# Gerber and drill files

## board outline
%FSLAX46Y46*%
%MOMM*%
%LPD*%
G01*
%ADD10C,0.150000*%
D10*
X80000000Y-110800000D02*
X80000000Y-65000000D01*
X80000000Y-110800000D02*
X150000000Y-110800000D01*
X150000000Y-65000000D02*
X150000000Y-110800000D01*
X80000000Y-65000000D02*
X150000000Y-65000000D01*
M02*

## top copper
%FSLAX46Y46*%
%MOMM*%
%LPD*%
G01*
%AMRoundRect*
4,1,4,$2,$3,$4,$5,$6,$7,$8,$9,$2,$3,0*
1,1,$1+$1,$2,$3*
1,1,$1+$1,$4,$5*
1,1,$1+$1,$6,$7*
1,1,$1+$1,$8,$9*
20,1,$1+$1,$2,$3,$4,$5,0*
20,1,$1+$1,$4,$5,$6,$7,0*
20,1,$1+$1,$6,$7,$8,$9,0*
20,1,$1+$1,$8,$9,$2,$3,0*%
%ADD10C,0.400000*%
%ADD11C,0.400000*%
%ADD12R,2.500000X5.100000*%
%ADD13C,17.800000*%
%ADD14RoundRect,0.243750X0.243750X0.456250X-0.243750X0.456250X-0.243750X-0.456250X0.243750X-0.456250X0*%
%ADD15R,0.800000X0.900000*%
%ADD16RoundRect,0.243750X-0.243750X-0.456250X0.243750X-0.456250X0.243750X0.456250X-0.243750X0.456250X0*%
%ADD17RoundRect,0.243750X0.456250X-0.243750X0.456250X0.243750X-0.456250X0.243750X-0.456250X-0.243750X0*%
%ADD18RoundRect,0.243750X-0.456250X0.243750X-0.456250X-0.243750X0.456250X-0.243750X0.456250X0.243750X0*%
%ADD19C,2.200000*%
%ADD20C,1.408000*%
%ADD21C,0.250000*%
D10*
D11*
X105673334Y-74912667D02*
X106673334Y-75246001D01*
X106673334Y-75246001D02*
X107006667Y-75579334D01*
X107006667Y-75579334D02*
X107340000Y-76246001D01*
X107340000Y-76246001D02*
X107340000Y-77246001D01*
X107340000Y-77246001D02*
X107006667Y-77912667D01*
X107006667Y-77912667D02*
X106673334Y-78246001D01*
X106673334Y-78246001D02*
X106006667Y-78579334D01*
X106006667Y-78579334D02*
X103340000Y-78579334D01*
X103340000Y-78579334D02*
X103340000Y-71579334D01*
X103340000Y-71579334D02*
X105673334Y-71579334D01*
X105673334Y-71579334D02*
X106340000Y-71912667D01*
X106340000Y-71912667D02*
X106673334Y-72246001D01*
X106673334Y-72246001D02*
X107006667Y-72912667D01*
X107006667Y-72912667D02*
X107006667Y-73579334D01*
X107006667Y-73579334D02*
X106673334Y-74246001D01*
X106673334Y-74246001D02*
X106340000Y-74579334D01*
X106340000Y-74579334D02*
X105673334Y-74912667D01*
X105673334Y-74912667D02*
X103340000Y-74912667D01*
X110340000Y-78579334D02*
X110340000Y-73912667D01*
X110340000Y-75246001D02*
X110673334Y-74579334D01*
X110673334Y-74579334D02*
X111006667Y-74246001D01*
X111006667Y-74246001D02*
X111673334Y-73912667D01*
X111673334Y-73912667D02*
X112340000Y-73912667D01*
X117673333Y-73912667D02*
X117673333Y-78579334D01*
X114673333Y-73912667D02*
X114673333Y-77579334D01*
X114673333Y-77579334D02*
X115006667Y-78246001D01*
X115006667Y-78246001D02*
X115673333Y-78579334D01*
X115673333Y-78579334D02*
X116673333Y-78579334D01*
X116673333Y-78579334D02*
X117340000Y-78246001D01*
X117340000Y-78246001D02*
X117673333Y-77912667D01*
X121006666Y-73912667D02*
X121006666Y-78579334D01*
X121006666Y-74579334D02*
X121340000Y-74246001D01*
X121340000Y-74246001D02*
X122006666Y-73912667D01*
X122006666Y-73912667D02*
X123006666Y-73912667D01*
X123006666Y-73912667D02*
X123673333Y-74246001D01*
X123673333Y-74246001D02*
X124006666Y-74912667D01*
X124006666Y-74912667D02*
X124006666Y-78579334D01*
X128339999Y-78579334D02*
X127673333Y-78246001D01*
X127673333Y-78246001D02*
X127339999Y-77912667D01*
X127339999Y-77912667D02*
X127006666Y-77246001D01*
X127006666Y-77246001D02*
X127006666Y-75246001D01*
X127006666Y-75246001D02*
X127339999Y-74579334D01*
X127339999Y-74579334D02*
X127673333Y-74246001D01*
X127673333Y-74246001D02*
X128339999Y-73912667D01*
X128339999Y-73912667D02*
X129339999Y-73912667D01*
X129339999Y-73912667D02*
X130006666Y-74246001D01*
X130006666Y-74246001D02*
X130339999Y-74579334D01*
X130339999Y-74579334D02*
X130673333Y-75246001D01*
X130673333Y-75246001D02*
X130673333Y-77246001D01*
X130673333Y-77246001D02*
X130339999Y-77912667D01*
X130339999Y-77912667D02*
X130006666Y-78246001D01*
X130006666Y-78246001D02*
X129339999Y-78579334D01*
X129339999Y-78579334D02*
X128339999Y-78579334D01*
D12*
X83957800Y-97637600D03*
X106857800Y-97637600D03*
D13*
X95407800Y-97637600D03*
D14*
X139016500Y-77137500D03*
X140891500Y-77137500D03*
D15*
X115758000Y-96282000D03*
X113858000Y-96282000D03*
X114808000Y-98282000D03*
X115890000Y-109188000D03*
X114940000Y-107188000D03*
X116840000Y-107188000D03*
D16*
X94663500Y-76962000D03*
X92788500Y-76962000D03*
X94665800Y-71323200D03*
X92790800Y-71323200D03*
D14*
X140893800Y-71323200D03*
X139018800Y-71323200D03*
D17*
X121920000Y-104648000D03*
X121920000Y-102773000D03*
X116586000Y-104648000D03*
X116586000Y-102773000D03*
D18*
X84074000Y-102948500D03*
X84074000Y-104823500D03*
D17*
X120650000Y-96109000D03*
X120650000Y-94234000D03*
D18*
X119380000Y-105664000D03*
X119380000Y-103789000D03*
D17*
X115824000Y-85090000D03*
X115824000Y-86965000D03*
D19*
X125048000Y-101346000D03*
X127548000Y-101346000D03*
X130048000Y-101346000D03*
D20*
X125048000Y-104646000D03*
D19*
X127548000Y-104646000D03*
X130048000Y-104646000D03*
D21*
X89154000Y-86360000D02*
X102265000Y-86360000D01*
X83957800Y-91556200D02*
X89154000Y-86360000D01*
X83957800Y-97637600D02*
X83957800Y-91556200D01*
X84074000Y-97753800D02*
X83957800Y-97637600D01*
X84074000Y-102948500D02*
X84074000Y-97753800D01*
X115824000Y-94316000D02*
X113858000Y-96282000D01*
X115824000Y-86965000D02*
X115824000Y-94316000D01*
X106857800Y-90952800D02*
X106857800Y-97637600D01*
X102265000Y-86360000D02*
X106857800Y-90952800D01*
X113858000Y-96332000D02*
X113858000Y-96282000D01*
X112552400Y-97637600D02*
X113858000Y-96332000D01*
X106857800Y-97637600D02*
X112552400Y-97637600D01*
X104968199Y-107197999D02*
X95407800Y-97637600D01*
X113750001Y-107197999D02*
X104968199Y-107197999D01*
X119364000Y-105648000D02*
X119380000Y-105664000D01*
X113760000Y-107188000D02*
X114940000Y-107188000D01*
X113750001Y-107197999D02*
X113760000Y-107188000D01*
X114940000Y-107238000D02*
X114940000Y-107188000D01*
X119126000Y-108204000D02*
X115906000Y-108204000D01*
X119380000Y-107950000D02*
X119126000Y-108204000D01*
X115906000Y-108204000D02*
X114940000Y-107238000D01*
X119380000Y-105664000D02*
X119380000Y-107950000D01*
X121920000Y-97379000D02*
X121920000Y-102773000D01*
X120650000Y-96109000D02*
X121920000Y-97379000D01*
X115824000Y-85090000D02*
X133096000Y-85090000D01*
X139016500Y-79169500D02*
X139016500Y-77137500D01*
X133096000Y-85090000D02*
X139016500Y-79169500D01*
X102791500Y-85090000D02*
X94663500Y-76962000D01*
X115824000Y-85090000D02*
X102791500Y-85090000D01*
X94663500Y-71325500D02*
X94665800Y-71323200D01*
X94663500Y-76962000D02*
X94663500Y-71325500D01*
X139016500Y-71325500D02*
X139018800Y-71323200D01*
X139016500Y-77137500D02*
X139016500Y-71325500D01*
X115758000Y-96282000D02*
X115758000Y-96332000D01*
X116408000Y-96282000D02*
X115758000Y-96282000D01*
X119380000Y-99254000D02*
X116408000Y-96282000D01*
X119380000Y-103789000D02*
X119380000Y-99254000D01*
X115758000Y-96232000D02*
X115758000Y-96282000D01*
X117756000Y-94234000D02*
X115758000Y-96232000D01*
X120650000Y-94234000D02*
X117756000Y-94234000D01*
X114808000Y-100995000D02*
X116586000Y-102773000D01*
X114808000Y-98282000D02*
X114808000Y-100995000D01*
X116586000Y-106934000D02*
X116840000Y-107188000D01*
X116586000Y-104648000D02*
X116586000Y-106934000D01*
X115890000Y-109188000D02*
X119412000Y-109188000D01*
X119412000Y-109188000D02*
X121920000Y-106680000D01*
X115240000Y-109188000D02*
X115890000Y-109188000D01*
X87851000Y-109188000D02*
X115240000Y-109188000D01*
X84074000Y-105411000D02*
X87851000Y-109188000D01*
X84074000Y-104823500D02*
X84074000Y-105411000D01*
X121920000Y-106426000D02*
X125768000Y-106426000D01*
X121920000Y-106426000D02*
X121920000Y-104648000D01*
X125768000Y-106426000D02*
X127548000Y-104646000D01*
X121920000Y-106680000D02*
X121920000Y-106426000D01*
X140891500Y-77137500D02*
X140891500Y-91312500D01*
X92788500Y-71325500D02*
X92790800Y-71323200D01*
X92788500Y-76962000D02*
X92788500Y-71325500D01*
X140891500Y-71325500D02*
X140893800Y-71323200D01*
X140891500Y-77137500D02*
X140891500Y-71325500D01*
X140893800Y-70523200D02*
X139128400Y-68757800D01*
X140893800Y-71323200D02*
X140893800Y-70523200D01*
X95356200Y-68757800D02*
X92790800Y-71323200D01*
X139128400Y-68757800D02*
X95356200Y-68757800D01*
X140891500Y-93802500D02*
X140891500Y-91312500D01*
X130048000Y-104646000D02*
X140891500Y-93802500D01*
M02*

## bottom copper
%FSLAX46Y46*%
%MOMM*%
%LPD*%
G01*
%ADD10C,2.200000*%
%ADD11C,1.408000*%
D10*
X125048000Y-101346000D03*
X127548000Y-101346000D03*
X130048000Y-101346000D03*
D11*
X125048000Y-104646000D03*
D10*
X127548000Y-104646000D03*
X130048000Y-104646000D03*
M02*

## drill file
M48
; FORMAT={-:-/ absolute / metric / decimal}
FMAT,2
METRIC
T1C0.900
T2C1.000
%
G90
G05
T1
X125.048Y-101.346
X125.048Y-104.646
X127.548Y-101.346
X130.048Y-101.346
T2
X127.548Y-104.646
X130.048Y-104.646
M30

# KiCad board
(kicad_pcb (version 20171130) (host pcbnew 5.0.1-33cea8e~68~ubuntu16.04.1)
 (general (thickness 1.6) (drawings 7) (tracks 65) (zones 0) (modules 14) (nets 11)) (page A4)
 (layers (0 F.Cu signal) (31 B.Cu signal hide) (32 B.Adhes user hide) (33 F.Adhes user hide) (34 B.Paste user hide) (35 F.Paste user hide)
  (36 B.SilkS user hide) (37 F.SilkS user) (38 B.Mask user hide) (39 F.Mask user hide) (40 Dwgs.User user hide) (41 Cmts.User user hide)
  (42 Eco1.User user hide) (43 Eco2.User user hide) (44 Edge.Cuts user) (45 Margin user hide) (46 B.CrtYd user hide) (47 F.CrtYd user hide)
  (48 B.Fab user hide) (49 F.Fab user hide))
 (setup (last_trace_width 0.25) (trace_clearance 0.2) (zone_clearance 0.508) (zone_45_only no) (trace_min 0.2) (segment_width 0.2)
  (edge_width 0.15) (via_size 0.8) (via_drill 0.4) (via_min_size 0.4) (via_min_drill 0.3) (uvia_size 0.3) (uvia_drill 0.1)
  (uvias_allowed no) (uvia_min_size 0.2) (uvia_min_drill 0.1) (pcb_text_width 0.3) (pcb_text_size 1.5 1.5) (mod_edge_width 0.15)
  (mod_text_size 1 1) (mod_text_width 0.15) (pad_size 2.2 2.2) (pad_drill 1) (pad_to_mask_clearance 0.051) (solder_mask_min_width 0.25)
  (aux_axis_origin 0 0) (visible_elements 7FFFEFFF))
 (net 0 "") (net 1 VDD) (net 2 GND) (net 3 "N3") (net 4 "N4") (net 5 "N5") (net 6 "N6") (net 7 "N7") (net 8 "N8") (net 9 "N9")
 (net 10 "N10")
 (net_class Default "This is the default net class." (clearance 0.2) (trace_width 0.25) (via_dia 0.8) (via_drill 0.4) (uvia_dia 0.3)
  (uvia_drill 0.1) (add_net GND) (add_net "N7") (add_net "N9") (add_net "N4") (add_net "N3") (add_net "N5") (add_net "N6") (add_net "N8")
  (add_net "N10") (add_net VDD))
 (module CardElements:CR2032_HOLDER (layer F.Cu) (at 95.4078 97.6376)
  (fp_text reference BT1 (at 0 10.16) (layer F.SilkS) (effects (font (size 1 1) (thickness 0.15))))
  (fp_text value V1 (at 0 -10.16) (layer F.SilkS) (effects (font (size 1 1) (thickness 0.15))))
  (pad 1 smd rect (at -11.45 0) (size 2.5 5.1) (layers F.Cu F.Paste F.Mask) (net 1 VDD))
  (pad 1 smd rect (at 11.45 0) (size 2.5 5.1) (layers F.Cu F.Paste F.Mask) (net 1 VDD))
  (pad 2 smd circle (at 0 0) (size 17.8 17.8) (layers F.Cu F.Paste F.Mask) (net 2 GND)))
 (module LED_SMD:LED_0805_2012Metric (layer F.Cu) (at 139.954 77.1375 180)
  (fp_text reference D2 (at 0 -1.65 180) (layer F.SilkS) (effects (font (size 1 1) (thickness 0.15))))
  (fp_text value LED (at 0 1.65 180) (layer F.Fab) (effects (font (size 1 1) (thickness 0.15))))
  (pad 2 smd roundrect (at 0.9375 0 180) (size 0.975 1.4) (layers F.Cu F.Paste F.Mask) (roundrect_rratio 0.25) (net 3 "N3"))
  (pad 1 smd roundrect (at -0.9375 0 180) (size 0.975 1.4) (layers F.Cu F.Paste F.Mask) (roundrect_rratio 0.25) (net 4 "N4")))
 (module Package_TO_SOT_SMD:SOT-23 (layer F.Cu) (at 114.808 97.282 270)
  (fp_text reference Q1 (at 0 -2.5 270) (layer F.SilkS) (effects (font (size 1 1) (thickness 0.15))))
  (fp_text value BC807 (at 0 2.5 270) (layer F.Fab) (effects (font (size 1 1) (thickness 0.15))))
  (pad 1 smd rect (at -1 -0.95 270) (size 0.9 0.8) (layers F.Cu F.Paste F.Mask) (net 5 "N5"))
  (pad 2 smd rect (at -1 0.95 270) (size 0.9 0.8) (layers F.Cu F.Paste F.Mask) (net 1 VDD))
  (pad 3 smd rect (at 1 0 270) (size 0.9 0.8) (layers F.Cu F.Paste F.Mask) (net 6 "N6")))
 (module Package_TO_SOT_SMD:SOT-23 (layer F.Cu) (at 115.89 108.188 270)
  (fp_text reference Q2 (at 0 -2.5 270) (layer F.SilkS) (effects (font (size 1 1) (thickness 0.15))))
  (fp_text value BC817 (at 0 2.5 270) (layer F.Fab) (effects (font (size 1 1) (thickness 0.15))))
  (pad 3 smd rect (at 1 0 270) (size 0.9 0.8) (layers F.Cu F.Paste F.Mask) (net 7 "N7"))
  (pad 2 smd rect (at -1 0.95 270) (size 0.9 0.8) (layers F.Cu F.Paste F.Mask) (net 2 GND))
  (pad 1 smd rect (at -1 -0.95 270) (size 0.9 0.8) (layers F.Cu F.Paste F.Mask) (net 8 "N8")))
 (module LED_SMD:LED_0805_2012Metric (layer F.Cu) (at 93.726 76.962)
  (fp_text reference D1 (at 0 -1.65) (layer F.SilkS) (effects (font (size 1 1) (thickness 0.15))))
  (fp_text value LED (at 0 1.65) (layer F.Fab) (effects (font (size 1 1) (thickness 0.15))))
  (pad 2 smd roundrect (at 0.9375 0) (size 0.975 1.4) (layers F.Cu F.Paste F.Mask) (roundrect_rratio 0.25) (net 3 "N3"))
  (pad 1 smd roundrect (at -0.9375 0) (size 0.975 1.4) (layers F.Cu F.Paste F.Mask) (roundrect_rratio 0.25) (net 4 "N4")))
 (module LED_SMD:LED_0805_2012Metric (layer F.Cu) (at 93.7283 71.3232)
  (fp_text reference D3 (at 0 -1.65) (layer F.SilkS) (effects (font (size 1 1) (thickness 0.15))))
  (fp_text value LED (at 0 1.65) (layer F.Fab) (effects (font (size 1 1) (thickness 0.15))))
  (pad 2 smd roundrect (at 0.9375 0) (size 0.975 1.4) (layers F.Cu F.Paste F.Mask) (roundrect_rratio 0.25) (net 3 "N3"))
  (pad 1 smd roundrect (at -0.9375 0) (size 0.975 1.4) (layers F.Cu F.Paste F.Mask) (roundrect_rratio 0.25) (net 4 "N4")))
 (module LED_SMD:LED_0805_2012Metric (layer F.Cu) (at 139.9563 71.3232 180)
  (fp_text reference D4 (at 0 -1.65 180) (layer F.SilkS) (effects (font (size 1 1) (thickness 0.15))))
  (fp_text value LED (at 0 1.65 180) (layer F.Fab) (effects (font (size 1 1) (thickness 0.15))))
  (pad 1 smd roundrect (at -0.9375 0 180) (size 0.975 1.4) (layers F.Cu F.Paste F.Mask) (roundrect_rratio 0.25) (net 4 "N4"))
  (pad 2 smd roundrect (at 0.9375 0 180) (size 0.975 1.4) (layers F.Cu F.Paste F.Mask) (roundrect_rratio 0.25) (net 3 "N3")))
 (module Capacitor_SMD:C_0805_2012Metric (layer F.Cu) (at 121.92 103.7105 90)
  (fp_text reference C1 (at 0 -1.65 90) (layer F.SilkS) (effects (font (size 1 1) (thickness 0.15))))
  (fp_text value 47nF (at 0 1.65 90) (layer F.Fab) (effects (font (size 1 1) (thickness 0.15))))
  (pad 1 smd roundrect (at -0.9375 0 90) (size 0.975 1.4) (layers F.Cu F.Paste F.Mask) (roundrect_rratio 0.25) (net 7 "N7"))
  (pad 2 smd roundrect (at 0.9375 0 90) (size 0.975 1.4) (layers F.Cu F.Paste F.Mask) (roundrect_rratio 0.25) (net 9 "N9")))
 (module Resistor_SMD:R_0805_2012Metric (layer F.Cu) (at 116.586 103.7105 90)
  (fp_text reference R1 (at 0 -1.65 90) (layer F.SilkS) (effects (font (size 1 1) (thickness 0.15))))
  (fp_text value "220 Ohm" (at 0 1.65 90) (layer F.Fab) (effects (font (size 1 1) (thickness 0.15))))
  (pad 1 smd roundrect (at -0.9375 0 90) (size 0.975 1.4) (layers F.Cu F.Paste F.Mask) (roundrect_rratio 0.25) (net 8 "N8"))
  (pad 2 smd roundrect (at 0.9375 0 90) (size 0.975 1.4) (layers F.Cu F.Paste F.Mask) (roundrect_rratio 0.25) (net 6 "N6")))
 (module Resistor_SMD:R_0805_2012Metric (layer F.Cu) (at 84.074 103.886 270)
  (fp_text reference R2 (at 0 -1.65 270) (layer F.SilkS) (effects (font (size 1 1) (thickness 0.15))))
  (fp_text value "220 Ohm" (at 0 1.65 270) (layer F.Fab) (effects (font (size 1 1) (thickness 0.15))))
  (pad 1 smd roundrect (at -0.9375 0 270) (size 0.975 1.4) (layers F.Cu F.Paste F.Mask) (roundrect_rratio 0.25) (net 1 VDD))
  (pad 2 smd roundrect (at 0.9375 0 270) (size 0.975 1.4) (layers F.Cu F.Paste F.Mask) (roundrect_rratio 0.25) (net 7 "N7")))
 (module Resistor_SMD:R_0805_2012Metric (layer F.Cu) (at 120.65 95.1715 90)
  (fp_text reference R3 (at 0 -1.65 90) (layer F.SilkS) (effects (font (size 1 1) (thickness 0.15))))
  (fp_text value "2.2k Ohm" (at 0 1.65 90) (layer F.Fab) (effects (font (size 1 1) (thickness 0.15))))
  (pad 1 smd roundrect (at -0.9375 0 90) (size 0.975 1.4) (layers F.Cu F.Paste F.Mask) (roundrect_rratio 0.25) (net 9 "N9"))
  (pad 2 smd roundrect (at 0.9375 0 90) (size 0.975 1.4) (layers F.Cu F.Paste F.Mask) (roundrect_rratio 0.25) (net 5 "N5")))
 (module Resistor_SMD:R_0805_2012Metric (layer F.Cu) (at 119.38 104.7265 270)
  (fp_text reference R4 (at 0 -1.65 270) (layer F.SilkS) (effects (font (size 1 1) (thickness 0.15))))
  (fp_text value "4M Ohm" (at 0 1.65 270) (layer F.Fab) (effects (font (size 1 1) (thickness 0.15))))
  (pad 2 smd roundrect (at 0.9375 0 270) (size 0.975 1.4) (layers F.Cu F.Paste F.Mask) (roundrect_rratio 0.25) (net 2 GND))
  (pad 1 smd roundrect (at -0.9375 0 270) (size 0.975 1.4) (layers F.Cu F.Paste F.Mask) (roundrect_rratio 0.25) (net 5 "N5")))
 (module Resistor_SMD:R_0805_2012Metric (layer F.Cu) (at 115.824 86.0275 90)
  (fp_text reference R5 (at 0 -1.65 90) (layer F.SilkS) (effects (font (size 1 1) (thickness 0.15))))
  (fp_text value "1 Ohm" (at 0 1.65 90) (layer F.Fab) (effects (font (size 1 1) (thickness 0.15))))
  (pad 2 smd roundrect (at 0.9375 0 90) (size 0.975 1.4) (layers F.Cu F.Paste F.Mask) (roundrect_rratio 0.25) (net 3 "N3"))
  (pad 1 smd roundrect (at -0.9375 0 90) (size 0.975 1.4) (layers F.Cu F.Paste F.Mask) (roundrect_rratio 0.25) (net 1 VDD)))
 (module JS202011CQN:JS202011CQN (layer F.Cu) (at 127.548 102.996 180)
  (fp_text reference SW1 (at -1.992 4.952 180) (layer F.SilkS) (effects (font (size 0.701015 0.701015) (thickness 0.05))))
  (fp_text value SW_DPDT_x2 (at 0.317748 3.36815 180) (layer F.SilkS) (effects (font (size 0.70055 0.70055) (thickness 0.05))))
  (pad 6 thru_hole circle (at 2.5 1.65 270) (size 2.2 2.2) (drill 0.9) (layers *.Cu *.Mask))
  (pad 5 thru_hole circle (at 0 1.65 270) (size 2.2 2.2) (drill 0.9) (layers *.Cu *.Mask))
  (pad 4 thru_hole circle (at -2.5 1.65 270) (size 2.2 2.2) (drill 0.9) (layers *.Cu *.Mask))
  (pad 3 thru_hole circle (at 2.5 -1.65 270) (size 1.408 1.408) (drill 0.9) (layers *.Cu *.Mask) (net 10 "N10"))
  (pad 2 thru_hole circle (at 0 -1.65 270) (size 2.2 2.2) (drill 1) (layers *.Cu *.Mask) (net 7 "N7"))
  (pad 1 thru_hole circle (at -2.5 -1.65 270) (size 2.2 2.2) (drill 1) (layers *.Cu *.Mask) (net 4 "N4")))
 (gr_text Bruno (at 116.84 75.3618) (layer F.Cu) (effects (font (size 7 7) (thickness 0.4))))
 (gr_line (start 80 110.8) (end 80 65) (layer Edge.Cuts) (width 0.15))
 (gr_line (start 80 110.8) (end 150 110.8) (layer Edge.Cuts) (width 0.15))
 (gr_line (start 150 65) (end 150 110.8) (layer Edge.Cuts) (width 0.15))
 (gr_line (start 80 65) (end 150 65) (layer Edge.Cuts) (width 0.15))
 (segment (start 89.154 86.36) (end 102.265 86.36) (width 0.25) (layer F.Cu) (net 1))
 (segment (start 83.9578 91.5562) (end 89.154 86.36) (width 0.25) (layer F.Cu) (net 1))
 (segment (start 83.9578 97.6376) (end 83.9578 91.5562) (width 0.25) (layer F.Cu) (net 1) (status 10))
 (segment (start 84.074 97.7538) (end 83.9578 97.6376) (width 0.25) (layer F.Cu) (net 1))
 (segment (start 84.074 102.9485) (end 84.074 97.7538) (width 0.25) (layer F.Cu) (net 1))
 (segment (start 115.824 94.316) (end 113.858 96.282) (width 0.25) (layer F.Cu) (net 1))
 (segment (start 115.824 86.965) (end 115.824 94.316) (width 0.25) (layer F.Cu) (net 1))
 (segment (start 106.8578 90.9528) (end 106.8578 97.6376) (width 0.25) (layer F.Cu) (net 1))
 (segment (start 102.265 86.36) (end 106.8578 90.9528) (width 0.25) (layer F.Cu) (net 1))
 (segment (start 113.858 96.332) (end 113.858 96.282) (width 0.25) (layer F.Cu) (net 1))
 (segment (start 112.5524 97.6376) (end 113.858 96.332) (width 0.25) (layer F.Cu) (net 1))
 (segment (start 106.8578 97.6376) (end 112.5524 97.6376) (width 0.25) (layer F.Cu) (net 1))
 (segment (start 104.968199 107.197999) (end 95.4078 97.6376) (width 0.25) (layer F.Cu) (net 2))
 (segment (start 113.750001 107.197999) (end 104.968199 107.197999) (width 0.25) (layer F.Cu) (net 2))
 (segment (start 119.364 105.648) (end 119.38 105.664) (width 0.25) (layer F.Cu) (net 2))
 (segment (start 113.76 107.188) (end 114.94 107.188) (width 0.25) (layer F.Cu) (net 2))
 (segment (start 113.750001 107.197999) (end 113.76 107.188) (width 0.25) (layer F.Cu) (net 2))
 (segment (start 114.94 107.238) (end 114.94 107.188) (width 0.25) (layer F.Cu) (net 2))
 (segment (start 119.126 108.204) (end 115.906 108.204) (width 0.25) (layer F.Cu) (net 2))
 (segment (start 119.38 107.95) (end 119.126 108.204) (width 0.25) (layer F.Cu) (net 2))
 (segment (start 115.906 108.204) (end 114.94 107.238) (width 0.25) (layer F.Cu) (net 2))
 (segment (start 119.38 105.664) (end 119.38 107.95) (width 0.25) (layer F.Cu) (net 2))
 (segment (start 121.92 97.379) (end 121.92 102.773) (width 0.25) (layer F.Cu) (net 9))
 (segment (start 120.65 96.109) (end 121.92 97.379) (width 0.25) (layer F.Cu) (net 9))
 (segment (start 115.824 85.09) (end 133.096 85.09) (width 0.25) (layer F.Cu) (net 3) (status 10))
 (segment (start 139.0165 79.1695) (end 139.0165 77.1375) (width 0.25) (layer F.Cu) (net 3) (status 20))
 (segment (start 133.096 85.09) (end 139.0165 79.1695) (width 0.25) (layer F.Cu) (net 3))
 (segment (start 102.7915 85.09) (end 94.6635 76.962) (width 0.25) (layer F.Cu) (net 3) (status 20))
 (segment (start 115.824 85.09) (end 102.7915 85.09) (width 0.25) (layer F.Cu) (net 3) (status 10))
 (segment (start 94.6635 71.3255) (end 94.6658 71.3232) (width 0.25) (layer F.Cu) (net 3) (status 30))
 (segment (start 94.6635 76.962) (end 94.6635 71.3255) (width 0.25) (layer F.Cu) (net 3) (status 30))
 (segment (start 139.0165 71.3255) (end 139.0188 71.3232) (width 0.25) (layer F.Cu) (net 3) (status 30))
 (segment (start 139.0165 77.1375) (end 139.0165 71.3255) (width 0.25) (layer F.Cu) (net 3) (status 30))
 (segment (start 115.758 96.282) (end 115.758 96.332) (width 0.25) (layer F.Cu) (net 5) (status 30))
 (segment (start 116.408 96.282) (end 115.758 96.282) (width 0.25) (layer F.Cu) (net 5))
 (segment (start 119.38 99.254) (end 116.408 96.282) (width 0.25) (layer F.Cu) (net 5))
 (segment (start 119.38 103.789) (end 119.38 99.254) (width 0.25) (layer F.Cu) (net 5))
 (segment (start 115.758 96.232) (end 115.758 96.282) (width 0.25) (layer F.Cu) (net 5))
 (segment (start 117.756 94.234) (end 115.758 96.232) (width 0.25) (layer F.Cu) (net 5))
 (segment (start 120.65 94.234) (end 117.756 94.234) (width 0.25) (layer F.Cu) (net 5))
 (segment (start 114.808 100.995) (end 116.586 102.773) (width 0.25) (layer F.Cu) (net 6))
 (segment (start 114.808 98.282) (end 114.808 100.995) (width 0.25) (layer F.Cu) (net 6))
 (segment (start 116.586 106.934) (end 116.84 107.188) (width 0.25) (layer F.Cu) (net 8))
 (segment (start 116.586 104.648) (end 116.586 106.934) (width 0.25) (layer F.Cu) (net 8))
 (segment (start 115.89 109.188) (end 119.412 109.188) (width 0.25) (layer F.Cu) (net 7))
 (segment (start 119.412 109.188) (end 121.92 106.68) (width 0.25) (layer F.Cu) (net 7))
 (segment (start 115.24 109.188) (end 115.89 109.188) (width 0.25) (layer F.Cu) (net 7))
 (segment (start 87.851 109.188) (end 115.24 109.188) (width 0.25) (layer F.Cu) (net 7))
 (segment (start 84.074 105.411) (end 87.851 109.188) (width 0.25) (layer F.Cu) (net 7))
 (segment (start 84.074 104.8235) (end 84.074 105.411) (width 0.25) (layer F.Cu) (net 7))
 (segment (start 121.92 106.426) (end 125.768 106.426) (width 0.25) (layer F.Cu) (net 7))
 (segment (start 121.92 106.426) (end 121.92 104.648) (width 0.25) (layer F.Cu) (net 7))
 (segment (start 125.768 106.426) (end 127.548 104.646) (width 0.25) (layer F.Cu) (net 7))
 (segment (start 121.92 106.68) (end 121.92 106.426) (width 0.25) (layer F.Cu) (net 7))
 (segment (start 140.8915 77.1375) (end 140.8915 91.3125) (width 0.25) (layer F.Cu) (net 4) (status 10))
 (segment (start 92.7885 71.3255) (end 92.7908 71.3232) (width 0.25) (layer F.Cu) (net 4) (status 30))
 (segment (start 92.7885 76.962) (end 92.7885 71.3255) (width 0.25) (layer F.Cu) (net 4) (status 30))
 (segment (start 140.8915 71.3255) (end 140.8938 71.3232) (width 0.25) (layer F.Cu) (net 4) (status 30))
 (segment (start 140.8915 77.1375) (end 140.8915 71.3255) (width 0.25) (layer F.Cu) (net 4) (status 30))
 (segment (start 140.8938 70.5232) (end 139.1284 68.7578) (width 0.25) (layer F.Cu) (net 4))
 (segment (start 140.8938 71.3232) (end 140.8938 70.5232) (width 0.25) (layer F.Cu) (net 4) (status 10))
 (segment (start 95.3562 68.7578) (end 92.7908 71.3232) (width 0.25) (layer F.Cu) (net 4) (status 20))
 (segment (start 139.1284 68.7578) (end 95.3562 68.7578) (width 0.25) (layer F.Cu) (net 4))
 (segment (start 140.8915 93.8025) (end 140.8915 91.3125) (width 0.25) (layer F.Cu) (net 4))
 (segment (start 130.048 104.646) (end 140.8915 93.8025) (width 0.25) (layer F.Cu) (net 4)))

